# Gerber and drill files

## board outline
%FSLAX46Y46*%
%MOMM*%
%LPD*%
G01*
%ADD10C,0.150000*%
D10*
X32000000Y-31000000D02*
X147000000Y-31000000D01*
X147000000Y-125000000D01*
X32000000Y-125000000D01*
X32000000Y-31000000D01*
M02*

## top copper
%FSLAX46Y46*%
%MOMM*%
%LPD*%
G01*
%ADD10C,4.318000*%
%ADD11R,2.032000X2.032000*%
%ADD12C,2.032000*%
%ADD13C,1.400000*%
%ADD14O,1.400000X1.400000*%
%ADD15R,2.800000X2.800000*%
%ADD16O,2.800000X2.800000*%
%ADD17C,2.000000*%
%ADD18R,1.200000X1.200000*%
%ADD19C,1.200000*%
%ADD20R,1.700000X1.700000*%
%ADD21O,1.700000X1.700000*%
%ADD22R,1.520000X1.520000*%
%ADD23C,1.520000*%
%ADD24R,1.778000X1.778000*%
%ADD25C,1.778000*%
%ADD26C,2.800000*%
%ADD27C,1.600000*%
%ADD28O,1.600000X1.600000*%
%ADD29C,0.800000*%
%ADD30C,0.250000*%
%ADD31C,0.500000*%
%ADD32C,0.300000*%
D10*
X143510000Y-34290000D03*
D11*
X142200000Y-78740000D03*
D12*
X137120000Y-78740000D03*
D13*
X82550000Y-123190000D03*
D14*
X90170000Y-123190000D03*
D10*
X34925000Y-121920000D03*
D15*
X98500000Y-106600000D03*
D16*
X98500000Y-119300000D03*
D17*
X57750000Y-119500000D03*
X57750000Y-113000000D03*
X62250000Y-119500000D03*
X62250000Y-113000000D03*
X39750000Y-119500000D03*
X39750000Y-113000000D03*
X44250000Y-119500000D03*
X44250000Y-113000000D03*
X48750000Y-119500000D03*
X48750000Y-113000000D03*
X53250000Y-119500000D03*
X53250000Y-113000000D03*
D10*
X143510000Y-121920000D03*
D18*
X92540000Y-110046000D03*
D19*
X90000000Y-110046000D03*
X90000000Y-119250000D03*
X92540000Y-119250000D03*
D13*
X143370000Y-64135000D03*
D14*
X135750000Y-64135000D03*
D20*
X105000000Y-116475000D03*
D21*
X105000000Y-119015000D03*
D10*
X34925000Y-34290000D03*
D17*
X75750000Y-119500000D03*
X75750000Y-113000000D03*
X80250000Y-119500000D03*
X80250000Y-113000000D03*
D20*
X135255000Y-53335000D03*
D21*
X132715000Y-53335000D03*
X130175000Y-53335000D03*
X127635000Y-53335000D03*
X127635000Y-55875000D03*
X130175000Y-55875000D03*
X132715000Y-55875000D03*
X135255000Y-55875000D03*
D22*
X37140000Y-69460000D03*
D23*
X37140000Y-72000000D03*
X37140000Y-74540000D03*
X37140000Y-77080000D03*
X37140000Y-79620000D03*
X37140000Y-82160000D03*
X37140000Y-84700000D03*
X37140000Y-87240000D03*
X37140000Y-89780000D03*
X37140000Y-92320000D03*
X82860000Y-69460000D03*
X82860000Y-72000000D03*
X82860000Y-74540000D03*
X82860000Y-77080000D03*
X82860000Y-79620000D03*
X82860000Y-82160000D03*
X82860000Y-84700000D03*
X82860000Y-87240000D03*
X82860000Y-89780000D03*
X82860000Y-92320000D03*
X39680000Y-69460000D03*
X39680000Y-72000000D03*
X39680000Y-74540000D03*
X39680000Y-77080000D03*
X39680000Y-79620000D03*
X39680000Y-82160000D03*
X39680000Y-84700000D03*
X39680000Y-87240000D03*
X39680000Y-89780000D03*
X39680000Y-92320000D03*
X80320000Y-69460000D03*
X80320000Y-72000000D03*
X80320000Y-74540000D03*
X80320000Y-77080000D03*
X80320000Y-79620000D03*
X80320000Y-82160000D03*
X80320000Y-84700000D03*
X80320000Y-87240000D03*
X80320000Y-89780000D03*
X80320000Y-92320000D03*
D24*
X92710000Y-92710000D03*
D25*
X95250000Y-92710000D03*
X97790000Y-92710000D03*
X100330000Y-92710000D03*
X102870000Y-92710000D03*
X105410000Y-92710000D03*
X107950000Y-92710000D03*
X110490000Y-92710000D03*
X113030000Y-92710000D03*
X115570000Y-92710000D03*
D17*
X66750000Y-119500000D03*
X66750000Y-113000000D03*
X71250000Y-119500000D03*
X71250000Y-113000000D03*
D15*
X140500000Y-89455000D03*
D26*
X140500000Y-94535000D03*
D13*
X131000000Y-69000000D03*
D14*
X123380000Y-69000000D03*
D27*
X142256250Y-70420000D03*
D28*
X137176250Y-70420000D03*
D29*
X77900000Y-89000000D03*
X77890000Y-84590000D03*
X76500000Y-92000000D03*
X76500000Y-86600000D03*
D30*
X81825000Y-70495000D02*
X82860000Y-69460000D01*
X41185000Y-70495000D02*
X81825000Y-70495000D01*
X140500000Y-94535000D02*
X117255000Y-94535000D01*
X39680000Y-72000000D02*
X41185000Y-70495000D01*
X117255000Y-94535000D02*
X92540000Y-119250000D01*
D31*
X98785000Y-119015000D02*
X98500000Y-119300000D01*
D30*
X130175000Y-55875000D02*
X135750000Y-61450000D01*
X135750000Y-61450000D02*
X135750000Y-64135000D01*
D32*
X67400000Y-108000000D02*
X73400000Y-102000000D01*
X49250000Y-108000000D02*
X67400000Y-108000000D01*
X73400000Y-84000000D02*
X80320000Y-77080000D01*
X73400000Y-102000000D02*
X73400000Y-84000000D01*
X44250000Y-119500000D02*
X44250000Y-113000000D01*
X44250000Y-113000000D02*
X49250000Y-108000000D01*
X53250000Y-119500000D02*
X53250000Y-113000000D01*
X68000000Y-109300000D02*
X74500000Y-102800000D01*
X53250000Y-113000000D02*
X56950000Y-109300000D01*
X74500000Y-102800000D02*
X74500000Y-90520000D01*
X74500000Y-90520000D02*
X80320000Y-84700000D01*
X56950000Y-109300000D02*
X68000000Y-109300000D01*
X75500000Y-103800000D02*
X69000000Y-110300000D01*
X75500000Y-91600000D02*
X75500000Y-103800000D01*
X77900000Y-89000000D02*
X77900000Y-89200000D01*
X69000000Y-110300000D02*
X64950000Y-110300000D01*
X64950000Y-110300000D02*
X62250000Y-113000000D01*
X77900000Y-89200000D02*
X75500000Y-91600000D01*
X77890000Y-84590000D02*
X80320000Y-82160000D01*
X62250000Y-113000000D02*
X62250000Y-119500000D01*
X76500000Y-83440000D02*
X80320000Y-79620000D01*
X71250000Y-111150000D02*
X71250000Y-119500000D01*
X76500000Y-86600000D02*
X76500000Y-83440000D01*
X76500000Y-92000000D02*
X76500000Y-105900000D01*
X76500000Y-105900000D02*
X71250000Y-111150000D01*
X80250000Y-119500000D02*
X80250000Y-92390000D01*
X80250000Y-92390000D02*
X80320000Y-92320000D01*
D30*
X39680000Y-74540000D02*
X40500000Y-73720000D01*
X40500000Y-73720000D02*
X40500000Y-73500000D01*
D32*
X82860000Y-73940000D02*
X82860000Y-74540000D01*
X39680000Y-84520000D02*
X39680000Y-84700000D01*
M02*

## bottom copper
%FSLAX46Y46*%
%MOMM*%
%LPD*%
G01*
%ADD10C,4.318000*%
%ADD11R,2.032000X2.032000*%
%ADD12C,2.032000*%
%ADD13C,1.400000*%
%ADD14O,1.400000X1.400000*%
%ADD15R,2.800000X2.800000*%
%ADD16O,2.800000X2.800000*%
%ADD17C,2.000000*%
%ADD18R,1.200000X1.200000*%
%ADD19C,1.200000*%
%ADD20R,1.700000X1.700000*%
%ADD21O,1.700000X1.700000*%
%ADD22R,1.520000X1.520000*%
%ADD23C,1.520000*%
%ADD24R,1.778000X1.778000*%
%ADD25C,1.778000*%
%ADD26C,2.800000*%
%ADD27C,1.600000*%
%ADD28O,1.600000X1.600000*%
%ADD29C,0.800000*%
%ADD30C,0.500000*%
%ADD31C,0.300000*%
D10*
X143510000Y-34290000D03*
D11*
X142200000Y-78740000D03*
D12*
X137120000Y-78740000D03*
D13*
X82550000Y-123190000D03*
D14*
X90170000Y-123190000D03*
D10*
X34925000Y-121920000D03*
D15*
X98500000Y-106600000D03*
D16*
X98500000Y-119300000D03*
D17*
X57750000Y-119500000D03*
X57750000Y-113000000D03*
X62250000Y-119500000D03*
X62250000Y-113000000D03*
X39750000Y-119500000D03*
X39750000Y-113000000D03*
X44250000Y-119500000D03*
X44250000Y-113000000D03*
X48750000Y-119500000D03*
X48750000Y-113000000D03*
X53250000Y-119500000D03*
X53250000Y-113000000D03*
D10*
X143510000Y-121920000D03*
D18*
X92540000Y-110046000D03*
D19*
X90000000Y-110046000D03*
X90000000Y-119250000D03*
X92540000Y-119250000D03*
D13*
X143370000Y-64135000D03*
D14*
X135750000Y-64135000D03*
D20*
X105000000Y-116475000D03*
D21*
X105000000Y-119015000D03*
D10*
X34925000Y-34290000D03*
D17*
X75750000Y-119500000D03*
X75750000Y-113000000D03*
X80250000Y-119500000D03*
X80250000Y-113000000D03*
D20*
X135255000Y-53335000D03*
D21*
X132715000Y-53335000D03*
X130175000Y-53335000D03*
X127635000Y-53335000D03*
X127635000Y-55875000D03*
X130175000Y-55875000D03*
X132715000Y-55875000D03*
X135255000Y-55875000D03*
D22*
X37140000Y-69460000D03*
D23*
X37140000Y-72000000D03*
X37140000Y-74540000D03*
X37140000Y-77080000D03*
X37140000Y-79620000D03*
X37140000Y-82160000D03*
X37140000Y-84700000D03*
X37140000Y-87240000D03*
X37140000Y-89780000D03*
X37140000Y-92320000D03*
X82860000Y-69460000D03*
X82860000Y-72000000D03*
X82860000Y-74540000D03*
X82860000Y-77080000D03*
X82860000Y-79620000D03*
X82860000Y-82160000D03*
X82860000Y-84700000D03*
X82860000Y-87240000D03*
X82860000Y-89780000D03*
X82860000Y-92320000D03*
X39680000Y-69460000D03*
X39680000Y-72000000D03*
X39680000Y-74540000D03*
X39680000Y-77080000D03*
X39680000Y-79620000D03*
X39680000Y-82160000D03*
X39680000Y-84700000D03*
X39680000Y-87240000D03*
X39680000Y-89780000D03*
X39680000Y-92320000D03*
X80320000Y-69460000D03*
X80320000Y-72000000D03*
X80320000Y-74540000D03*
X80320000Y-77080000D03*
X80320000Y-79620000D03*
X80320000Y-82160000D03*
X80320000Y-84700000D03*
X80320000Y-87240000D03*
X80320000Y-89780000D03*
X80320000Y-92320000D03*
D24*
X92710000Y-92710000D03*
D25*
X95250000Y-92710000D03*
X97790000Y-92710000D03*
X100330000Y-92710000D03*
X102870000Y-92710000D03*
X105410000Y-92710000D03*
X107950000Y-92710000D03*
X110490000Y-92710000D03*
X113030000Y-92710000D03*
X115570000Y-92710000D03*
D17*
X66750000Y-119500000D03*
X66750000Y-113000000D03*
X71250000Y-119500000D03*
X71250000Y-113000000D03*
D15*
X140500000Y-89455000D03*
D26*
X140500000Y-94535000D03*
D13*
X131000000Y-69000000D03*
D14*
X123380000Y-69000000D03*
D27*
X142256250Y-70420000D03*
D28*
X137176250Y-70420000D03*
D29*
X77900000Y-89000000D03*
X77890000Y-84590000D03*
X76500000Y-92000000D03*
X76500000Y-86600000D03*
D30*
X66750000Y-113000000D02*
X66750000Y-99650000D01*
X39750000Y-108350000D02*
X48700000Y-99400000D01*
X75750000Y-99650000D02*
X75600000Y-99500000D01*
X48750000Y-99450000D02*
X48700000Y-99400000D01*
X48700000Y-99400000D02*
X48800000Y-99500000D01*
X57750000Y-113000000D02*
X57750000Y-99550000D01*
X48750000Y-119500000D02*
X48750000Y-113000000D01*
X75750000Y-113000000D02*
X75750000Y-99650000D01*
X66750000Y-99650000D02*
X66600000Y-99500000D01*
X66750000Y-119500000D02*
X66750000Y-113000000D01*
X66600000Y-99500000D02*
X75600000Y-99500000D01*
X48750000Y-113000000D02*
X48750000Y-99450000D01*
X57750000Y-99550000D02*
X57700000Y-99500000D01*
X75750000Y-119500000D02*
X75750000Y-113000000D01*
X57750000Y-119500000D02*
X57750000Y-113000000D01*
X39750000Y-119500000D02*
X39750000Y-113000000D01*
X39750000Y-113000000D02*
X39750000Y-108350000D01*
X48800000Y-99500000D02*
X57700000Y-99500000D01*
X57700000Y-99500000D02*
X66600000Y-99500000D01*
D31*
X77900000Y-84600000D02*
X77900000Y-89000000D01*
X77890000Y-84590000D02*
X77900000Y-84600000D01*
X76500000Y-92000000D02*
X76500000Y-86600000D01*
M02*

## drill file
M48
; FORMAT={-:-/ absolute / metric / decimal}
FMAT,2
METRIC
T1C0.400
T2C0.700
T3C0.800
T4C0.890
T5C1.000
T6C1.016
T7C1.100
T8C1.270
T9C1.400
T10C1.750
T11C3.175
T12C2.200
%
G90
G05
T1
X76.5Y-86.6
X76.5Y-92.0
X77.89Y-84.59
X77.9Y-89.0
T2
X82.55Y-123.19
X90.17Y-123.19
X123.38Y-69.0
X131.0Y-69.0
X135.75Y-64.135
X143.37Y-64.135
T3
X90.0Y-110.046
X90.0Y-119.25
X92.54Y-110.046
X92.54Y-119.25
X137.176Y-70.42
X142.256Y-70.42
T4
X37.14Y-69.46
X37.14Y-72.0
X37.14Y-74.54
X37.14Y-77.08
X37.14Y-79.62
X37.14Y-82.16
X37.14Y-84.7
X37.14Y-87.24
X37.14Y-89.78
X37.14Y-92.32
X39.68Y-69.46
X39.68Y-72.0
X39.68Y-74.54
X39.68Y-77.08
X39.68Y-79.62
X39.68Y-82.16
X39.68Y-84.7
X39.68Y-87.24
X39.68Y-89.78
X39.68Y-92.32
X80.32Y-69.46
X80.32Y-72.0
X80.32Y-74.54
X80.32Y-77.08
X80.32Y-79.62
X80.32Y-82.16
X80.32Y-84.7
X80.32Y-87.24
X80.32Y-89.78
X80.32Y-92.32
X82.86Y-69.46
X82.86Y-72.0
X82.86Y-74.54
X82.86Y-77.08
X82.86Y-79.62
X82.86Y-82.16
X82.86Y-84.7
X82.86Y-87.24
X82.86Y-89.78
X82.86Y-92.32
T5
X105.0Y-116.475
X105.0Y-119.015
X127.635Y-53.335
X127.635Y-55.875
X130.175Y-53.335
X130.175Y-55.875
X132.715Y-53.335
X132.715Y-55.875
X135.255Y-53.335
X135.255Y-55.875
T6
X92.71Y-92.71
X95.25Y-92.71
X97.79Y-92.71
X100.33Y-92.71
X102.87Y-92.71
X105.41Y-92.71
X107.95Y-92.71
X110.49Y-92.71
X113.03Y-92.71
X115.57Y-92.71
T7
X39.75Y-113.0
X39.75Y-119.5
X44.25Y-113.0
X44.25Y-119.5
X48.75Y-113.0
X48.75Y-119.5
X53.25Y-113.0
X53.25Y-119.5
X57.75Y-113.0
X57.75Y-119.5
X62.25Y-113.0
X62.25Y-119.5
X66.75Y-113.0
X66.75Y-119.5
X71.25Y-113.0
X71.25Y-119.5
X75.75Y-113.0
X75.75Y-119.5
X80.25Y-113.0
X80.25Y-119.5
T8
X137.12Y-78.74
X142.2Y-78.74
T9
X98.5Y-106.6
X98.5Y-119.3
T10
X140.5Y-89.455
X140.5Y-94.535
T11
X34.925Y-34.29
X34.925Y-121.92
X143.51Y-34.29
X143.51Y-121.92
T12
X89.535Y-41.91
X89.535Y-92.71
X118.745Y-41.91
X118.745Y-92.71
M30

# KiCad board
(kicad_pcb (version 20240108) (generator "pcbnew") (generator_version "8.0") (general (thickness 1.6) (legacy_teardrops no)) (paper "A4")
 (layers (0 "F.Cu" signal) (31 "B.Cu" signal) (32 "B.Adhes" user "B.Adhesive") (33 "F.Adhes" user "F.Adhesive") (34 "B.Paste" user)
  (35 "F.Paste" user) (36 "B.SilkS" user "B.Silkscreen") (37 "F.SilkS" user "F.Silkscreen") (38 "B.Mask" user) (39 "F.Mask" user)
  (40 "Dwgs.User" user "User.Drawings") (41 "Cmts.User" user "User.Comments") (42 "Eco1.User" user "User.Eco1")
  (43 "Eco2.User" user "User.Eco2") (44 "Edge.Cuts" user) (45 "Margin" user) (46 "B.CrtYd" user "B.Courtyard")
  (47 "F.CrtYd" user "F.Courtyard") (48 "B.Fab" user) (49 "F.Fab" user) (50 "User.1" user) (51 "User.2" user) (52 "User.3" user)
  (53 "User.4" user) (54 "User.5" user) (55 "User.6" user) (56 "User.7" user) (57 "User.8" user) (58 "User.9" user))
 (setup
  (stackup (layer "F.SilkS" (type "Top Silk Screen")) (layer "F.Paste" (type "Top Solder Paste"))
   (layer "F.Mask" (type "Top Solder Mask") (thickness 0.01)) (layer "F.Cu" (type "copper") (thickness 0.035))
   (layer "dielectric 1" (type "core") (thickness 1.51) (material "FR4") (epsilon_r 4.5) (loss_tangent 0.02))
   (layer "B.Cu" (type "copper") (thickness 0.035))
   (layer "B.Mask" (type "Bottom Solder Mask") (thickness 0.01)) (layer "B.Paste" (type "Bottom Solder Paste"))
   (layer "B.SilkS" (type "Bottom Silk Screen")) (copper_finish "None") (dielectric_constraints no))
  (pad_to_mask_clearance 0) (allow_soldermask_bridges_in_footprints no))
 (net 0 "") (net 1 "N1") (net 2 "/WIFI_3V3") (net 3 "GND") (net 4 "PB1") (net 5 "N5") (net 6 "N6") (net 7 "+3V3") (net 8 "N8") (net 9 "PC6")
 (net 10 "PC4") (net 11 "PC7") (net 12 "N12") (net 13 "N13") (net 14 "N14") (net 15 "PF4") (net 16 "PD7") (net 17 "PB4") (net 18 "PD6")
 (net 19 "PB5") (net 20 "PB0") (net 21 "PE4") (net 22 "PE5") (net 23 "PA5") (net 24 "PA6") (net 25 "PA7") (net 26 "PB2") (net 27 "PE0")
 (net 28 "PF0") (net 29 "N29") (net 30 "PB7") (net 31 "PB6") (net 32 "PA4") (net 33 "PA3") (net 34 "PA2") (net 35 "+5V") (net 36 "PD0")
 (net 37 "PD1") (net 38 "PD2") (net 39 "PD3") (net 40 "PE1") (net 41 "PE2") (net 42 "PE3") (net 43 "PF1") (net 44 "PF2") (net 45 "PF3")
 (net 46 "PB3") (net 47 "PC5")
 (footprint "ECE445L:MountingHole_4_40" (layer "F.Cu") (at 143.51 34.29)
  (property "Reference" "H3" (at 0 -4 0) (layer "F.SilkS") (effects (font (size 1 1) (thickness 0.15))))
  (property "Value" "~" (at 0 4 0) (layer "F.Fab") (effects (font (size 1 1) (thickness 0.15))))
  (pad "1" thru_hole circle (at 0 0) (size 4.318 4.318) (drill 3.175) (layers "*.Cu" "*.Mask") (remove_unused_layers no) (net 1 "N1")))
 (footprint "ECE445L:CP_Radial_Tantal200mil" (layer "F.Cu") (at 142.2 78.74 180)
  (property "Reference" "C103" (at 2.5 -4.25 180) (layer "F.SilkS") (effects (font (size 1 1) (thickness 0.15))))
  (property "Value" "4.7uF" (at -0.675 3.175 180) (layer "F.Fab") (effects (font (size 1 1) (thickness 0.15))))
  (pad "1" thru_hole rect (at 0 0 180) (size 2.032 2.032) (drill 1.27) (layers "*.Cu" "*.Mask") (remove_unused_layers no)
   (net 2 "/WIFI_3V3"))
  (pad "2" thru_hole circle (at 5.08 0 180) (size 2.032 2.032) (drill 1.27) (layers "*.Cu" "*.Mask") (remove_unused_layers no) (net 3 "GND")))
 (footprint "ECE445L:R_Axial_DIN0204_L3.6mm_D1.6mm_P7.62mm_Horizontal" (layer "F.Cu") (at 82.55 123.19)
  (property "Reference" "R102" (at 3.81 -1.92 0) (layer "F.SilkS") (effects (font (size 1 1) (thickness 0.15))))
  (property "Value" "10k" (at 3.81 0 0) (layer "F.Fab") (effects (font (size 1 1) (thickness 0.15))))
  (pad "1" thru_hole circle (at 0 0) (size 1.4 1.4) (drill 0.7) (layers "*.Cu" "*.Mask") (remove_unused_layers no) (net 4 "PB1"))
  (pad "2" thru_hole oval (at 7.62 0) (size 1.4 1.4) (drill 0.7) (layers "*.Cu" "*.Mask") (remove_unused_layers no) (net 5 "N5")))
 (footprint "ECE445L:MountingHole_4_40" (layer "F.Cu") (at 34.925 121.92)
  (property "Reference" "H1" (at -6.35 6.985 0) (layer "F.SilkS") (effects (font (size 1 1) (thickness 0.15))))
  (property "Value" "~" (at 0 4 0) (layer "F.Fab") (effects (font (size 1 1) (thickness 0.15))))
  (pad "1" thru_hole circle (at 0 0) (size 4.318 4.318) (drill 3.175) (layers "*.Cu" "*.Mask") (remove_unused_layers no) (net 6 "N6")))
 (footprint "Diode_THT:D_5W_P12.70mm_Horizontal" (layer "F.Cu") (at 98.5 106.6 -90)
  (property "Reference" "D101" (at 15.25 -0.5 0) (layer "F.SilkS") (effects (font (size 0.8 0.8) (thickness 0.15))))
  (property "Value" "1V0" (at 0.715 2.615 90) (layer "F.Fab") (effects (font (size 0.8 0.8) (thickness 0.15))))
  (pad "1" thru_hole rect (at 0 0 270) (size 2.8 2.8) (drill 1.4) (layers "*.Cu" "*.Mask") (remove_unused_layers no) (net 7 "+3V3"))
  (pad "2" thru_hole oval (at 12.7 0 270) (size 2.8 2.8) (drill 1.4) (layers "*.Cu" "*.Mask") (remove_unused_layers no) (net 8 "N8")))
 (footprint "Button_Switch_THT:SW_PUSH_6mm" (layer "F.Cu") (at 57.75 119.5 90)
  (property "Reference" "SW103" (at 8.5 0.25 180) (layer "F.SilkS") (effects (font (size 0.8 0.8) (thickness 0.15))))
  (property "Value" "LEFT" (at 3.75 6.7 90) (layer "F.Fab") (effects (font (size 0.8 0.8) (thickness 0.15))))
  (pad "1" thru_hole circle (at 0 0 180) (size 2 2) (drill 1.1) (layers "*.Cu" "*.Mask") (remove_unused_layers no) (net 3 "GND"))
  (pad "1" thru_hole circle (at 6.5 0 180) (size 2 2) (drill 1.1) (layers "*.Cu" "*.Mask") (remove_unused_layers no) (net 3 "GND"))
  (pad "2" thru_hole circle (at 0 4.5 180) (size 2 2) (drill 1.1) (layers "*.Cu" "*.Mask") (remove_unused_layers no) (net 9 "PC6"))
  (pad "2" thru_hole circle (at 6.5 4.5 180) (size 2 2) (drill 1.1) (layers "*.Cu" "*.Mask") (remove_unused_layers no) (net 9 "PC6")))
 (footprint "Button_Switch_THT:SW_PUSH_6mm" (layer "F.Cu") (at 39.75 119.5 90)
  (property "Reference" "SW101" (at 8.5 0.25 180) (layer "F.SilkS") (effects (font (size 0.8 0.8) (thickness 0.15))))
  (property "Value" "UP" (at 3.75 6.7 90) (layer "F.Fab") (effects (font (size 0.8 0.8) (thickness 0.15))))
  (pad "1" thru_hole circle (at 0 0 180) (size 2 2) (drill 1.1) (layers "*.Cu" "*.Mask") (remove_unused_layers no) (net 3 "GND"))
  (pad "1" thru_hole circle (at 6.5 0 180) (size 2 2) (drill 1.1) (layers "*.Cu" "*.Mask") (remove_unused_layers no) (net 3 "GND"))
  (pad "2" thru_hole circle (at 0 4.5 180) (size 2 2) (drill 1.1) (layers "*.Cu" "*.Mask") (remove_unused_layers no) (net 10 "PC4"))
  (pad "2" thru_hole circle (at 6.5 4.5 180) (size 2 2) (drill 1.1) (layers "*.Cu" "*.Mask") (remove_unused_layers no) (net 10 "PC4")))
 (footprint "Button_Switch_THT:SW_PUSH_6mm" (layer "F.Cu") (at 48.75 119.5 90)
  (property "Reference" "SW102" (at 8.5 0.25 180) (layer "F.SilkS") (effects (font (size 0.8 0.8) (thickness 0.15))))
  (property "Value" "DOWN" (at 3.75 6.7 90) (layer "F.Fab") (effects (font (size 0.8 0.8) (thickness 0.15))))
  (pad "1" thru_hole circle (at 0 0 180) (size 2 2) (drill 1.1) (layers "*.Cu" "*.Mask") (remove_unused_layers no) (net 3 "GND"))
  (pad "1" thru_hole circle (at 6.5 0 180) (size 2 2) (drill 1.1) (layers "*.Cu" "*.Mask") (remove_unused_layers no) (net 3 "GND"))
  (pad "2" thru_hole circle (at 0 4.5 180) (size 2 2) (drill 1.1) (layers "*.Cu" "*.Mask") (remove_unused_layers no) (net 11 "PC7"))
  (pad "2" thru_hole circle (at 6.5 4.5 180) (size 2 2) (drill 1.1) (layers "*.Cu" "*.Mask") (remove_unused_layers no) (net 11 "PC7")))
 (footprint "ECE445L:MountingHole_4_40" (layer "F.Cu") (at 143.51 121.92)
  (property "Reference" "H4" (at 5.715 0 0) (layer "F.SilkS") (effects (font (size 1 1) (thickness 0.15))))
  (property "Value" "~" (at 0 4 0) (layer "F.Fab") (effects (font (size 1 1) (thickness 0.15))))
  (pad "1" thru_hole circle (at 0 0) (size 4.318 4.318) (drill 3.175) (layers "*.Cu" "*.Mask") (remove_unused_layers no) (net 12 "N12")))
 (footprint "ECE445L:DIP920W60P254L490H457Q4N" (layer "F.Cu") (at 91.27 114.648 -90)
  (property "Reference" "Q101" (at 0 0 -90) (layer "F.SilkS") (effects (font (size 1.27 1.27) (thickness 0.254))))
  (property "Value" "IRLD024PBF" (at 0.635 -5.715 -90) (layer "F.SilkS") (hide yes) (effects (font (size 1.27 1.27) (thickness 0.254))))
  (pad "1" thru_hole rect (at -4.602 -1.27 270) (size 1.2 1.2) (drill 0.8) (layers "*.Cu" "*.Mask") (remove_unused_layers no) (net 8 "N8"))
  (pad "2" thru_hole circle (at -4.602 1.27 270) (size 1.2 1.2) (drill 0.8) (layers "*.Cu" "*.Mask") (remove_unused_layers no) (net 8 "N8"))
  (pad "3" thru_hole circle (at 4.602 1.27 270) (size 1.2 1.2) (drill 0.8) (layers "*.Cu" "*.Mask") (remove_unused_layers no) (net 5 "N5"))
  (pad "4" thru_hole circle (at 4.602 -1.27 270) (size 1.2 1.2) (drill 0.8) (layers "*.Cu" "*.Mask") (remove_unused_layers no) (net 3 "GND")))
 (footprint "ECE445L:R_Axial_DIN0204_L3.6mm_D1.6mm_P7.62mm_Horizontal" (layer "F.Cu") (at 143.37 64.135 180)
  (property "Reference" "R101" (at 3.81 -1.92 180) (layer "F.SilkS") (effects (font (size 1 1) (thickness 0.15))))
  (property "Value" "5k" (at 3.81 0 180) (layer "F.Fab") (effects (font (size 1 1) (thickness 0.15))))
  (pad "1" thru_hole circle (at 0 0 180) (size 1.4 1.4) (drill 0.7) (layers "*.Cu" "*.Mask") (remove_unused_layers no) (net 2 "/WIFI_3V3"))
  (pad "2" thru_hole oval (at 7.62 0 180) (size 1.4 1.4) (drill 0.7) (layers "*.Cu" "*.Mask") (remove_unused_layers no) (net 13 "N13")))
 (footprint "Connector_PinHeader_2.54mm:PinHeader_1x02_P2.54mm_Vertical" (layer "F.Cu") (at 105 116.475)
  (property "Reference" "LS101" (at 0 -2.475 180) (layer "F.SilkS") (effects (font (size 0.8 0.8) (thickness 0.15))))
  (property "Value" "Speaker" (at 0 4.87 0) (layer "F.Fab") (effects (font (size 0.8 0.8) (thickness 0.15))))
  (pad "1" thru_hole rect (at 0 0) (size 1.7 1.7) (drill 1) (layers "*.Cu" "*.Mask") (remove_unused_layers no) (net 7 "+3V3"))
  (pad "2" thru_hole oval (at 0 2.54) (size 1.7 1.7) (drill 1) (layers "*.Cu" "*.Mask") (remove_unused_layers no) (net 8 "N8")))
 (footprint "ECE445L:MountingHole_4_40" (layer "F.Cu") (at 34.925 34.29)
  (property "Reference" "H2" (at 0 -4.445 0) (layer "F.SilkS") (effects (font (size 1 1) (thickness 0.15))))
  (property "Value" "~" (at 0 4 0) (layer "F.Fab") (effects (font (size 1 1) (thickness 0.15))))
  (pad "1" thru_hole circle (at 0 0) (size 4.318 4.318) (drill 3.175) (layers "*.Cu" "*.Mask") (remove_unused_layers no) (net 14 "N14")))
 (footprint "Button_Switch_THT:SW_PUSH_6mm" (layer "F.Cu") (at 75.75 119.5 90)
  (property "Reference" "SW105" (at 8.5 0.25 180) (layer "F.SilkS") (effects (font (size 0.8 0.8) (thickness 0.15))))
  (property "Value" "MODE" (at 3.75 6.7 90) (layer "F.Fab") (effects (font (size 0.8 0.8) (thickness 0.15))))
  (pad "1" thru_hole circle (at 0 0 180) (size 2 2) (drill 1.1) (layers "*.Cu" "*.Mask") (remove_unused_layers no) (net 3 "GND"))
  (pad "1" thru_hole circle (at 6.5 0 180) (size 2 2) (drill 1.1) (layers "*.Cu" "*.Mask") (remove_unused_layers no) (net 3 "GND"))
  (pad "2" thru_hole circle (at 0 4.5 180) (size 2 2) (drill 1.1) (layers "*.Cu" "*.Mask") (remove_unused_layers no) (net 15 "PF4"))
  (pad "2" thru_hole circle (at 6.5 4.5 180) (size 2 2) (drill 1.1) (layers "*.Cu" "*.Mask") (remove_unused_layers no) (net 15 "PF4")))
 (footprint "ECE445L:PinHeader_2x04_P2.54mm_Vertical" (layer "F.Cu") (at 135.255 53.335 -90)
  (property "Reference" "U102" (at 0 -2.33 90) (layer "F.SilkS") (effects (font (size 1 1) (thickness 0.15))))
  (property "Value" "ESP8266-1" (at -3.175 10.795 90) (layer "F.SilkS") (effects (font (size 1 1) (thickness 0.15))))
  (pad "1" thru_hole rect (at 0 0 270) (size 1.7 1.7) (drill 1) (layers "*.Cu" "*.Mask") (remove_unused_layers no) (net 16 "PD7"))
  (pad "2" thru_hole oval (at 0 2.54 270) (size 1.7 1.7) (drill 1) (layers "*.Cu" "*.Mask") (remove_unused_layers no) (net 2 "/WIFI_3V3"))
  (pad "3" thru_hole oval (at 0 5.08 270) (size 1.7 1.7) (drill 1) (layers "*.Cu" "*.Mask") (remove_unused_layers no) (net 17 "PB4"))
  (pad "4" thru_hole oval (at 0 7.62 270) (size 1.7 1.7) (drill 1) (layers "*.Cu" "*.Mask") (remove_unused_layers no) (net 3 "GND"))
  (pad "5" thru_hole oval (at 2.54 7.62 270) (size 1.7 1.7) (drill 1) (layers "*.Cu" "*.Mask") (remove_unused_layers no) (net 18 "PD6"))
  (pad "6" thru_hole oval (at 2.54 5.08 270) (size 1.7 1.7) (drill 1) (layers "*.Cu" "*.Mask") (remove_unused_layers no) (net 13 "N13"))
  (pad "7" thru_hole oval (at 2.54 2.54 270) (size 1.7 1.7) (drill 1) (layers "*.Cu" "*.Mask") (remove_unused_layers no) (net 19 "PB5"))
  (pad "8" thru_hole oval (at 2.54 0 270) (size 1.7 1.7) (drill 1) (layers "*.Cu" "*.Mask") (remove_unused_layers no) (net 2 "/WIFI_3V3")))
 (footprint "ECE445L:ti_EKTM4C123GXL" (layer "F.Cu") (at 60 72)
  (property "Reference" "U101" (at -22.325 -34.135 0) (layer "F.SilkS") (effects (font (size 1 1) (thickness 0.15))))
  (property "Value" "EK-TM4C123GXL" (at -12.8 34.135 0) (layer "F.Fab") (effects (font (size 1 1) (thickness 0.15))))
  (pad "J1_1" thru_hole rect (at -22.86 -2.54) (size 1.52 1.52) (drill 0.89) (layers "*.Cu" "*.Mask") (remove_unused_layers no)
   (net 7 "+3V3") (solder_mask_margin 0.102))
  (pad "J1_2" thru_hole circle (at -22.86 0) (size 1.52 1.52) (drill 0.89) (layers "*.Cu" "*.Mask") (remove_unused_layers no) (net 19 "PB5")
   (solder_mask_margin 0.102))
  (pad "J1_3" thru_hole circle (at -22.86 2.54) (size 1.52 1.52) (drill 0.89) (layers "*.Cu" "*.Mask") (remove_unused_layers no)
   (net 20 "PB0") (solder_mask_margin 0.102))
  (pad "J1_4" thru_hole circle (at -22.86 5.08) (size 1.52 1.52) (drill 0.89) (layers "*.Cu" "*.Mask") (remove_unused_layers no)
   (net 4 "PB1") (solder_mask_margin 0.102))
  (pad "J1_5" thru_hole circle (at -22.86 7.62) (size 1.52 1.52) (drill 0.89) (layers "*.Cu" "*.Mask") (remove_unused_layers no)
   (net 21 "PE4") (solder_mask_margin 0.102))
  (pad "J1_6" thru_hole circle (at -22.86 10.16) (size 1.52 1.52) (drill 0.89) (layers "*.Cu" "*.Mask") (remove_unused_layers no)
   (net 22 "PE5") (solder_mask_margin 0.102))
  (pad "J1_7" thru_hole circle (at -22.86 12.7) (size 1.52 1.52) (drill 0.89) (layers "*.Cu" "*.Mask") (remove_unused_layers no)
   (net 17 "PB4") (solder_mask_margin 0.102))
  (pad "J1_8" thru_hole circle (at -22.86 15.24) (size 1.52 1.52) (drill 0.89) (layers "*.Cu" "*.Mask") (remove_unused_layers no)
   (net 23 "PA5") (solder_mask_margin 0.102))
  (pad "J1_9" thru_hole circle (at -22.86 17.78) (size 1.52 1.52) (drill 0.89) (layers "*.Cu" "*.Mask") (remove_unused_layers no)
   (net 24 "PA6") (solder_mask_margin 0.102))
  (pad "J1_10" thru_hole circle (at -22.86 20.32) (size 1.52 1.52) (drill 0.89) (layers "*.Cu" "*.Mask") (remove_unused_layers no)
   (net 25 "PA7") (solder_mask_margin 0.102))
  (pad "J2_1" thru_hole circle (at 22.86 -2.54) (size 1.52 1.52) (drill 0.89) (layers "*.Cu" "*.Mask") (remove_unused_layers no)
   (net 3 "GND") (solder_mask_margin 0.102))
  (pad "J2_2" thru_hole circle (at 22.86 0) (size 1.52 1.52) (drill 0.89) (layers "*.Cu" "*.Mask") (remove_unused_layers no) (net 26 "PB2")
   (solder_mask_margin 0.102))
  (pad "J2_3" thru_hole circle (at 22.86 2.54) (size 1.52 1.52) (drill 0.89) (layers "*.Cu" "*.Mask") (remove_unused_layers no)
   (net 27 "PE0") (solder_mask_margin 0.102))
  (pad "J2_4" thru_hole circle (at 22.86 5.08) (size 1.52 1.52) (drill 0.89) (layers "*.Cu" "*.Mask") (remove_unused_layers no)
   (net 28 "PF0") (solder_mask_margin 0.102))
  (pad "J2_5" thru_hole circle (at 22.86 7.62) (size 1.52 1.52) (drill 0.89) (layers "*.Cu" "*.Mask") (remove_unused_layers no)
   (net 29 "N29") (solder_mask_margin 0.102))
  (pad "J2_6" thru_hole circle (at 22.86 10.16) (size 1.52 1.52) (drill 0.89) (layers "*.Cu" "*.Mask") (remove_unused_layers no)
   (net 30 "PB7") (solder_mask_margin 0.102))
  (pad "J2_7" thru_hole circle (at 22.86 12.7) (size 1.52 1.52) (drill 0.89) (layers "*.Cu" "*.Mask") (remove_unused_layers no)
   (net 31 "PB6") (solder_mask_margin 0.102))
  (pad "J2_8" thru_hole circle (at 22.86 15.24) (size 1.52 1.52) (drill 0.89) (layers "*.Cu" "*.Mask") (remove_unused_layers no)
   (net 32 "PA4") (solder_mask_margin 0.102))
  (pad "J2_9" thru_hole circle (at 22.86 17.78) (size 1.52 1.52) (drill 0.89) (layers "*.Cu" "*.Mask") (remove_unused_layers no)
   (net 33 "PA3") (solder_mask_margin 0.102))
  (pad "J2_10" thru_hole circle (at 22.86 20.32) (size 1.52 1.52) (drill 0.89) (layers "*.Cu" "*.Mask") (remove_unused_layers no)
   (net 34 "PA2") (solder_mask_margin 0.102))
  (pad "J3_1" thru_hole circle (at -20.32 -2.54) (size 1.52 1.52) (drill 0.89) (layers "*.Cu" "*.Mask") (remove_unused_layers no)
   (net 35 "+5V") (solder_mask_margin 0.102))
  (pad "J3_2" thru_hole circle (at -20.32 0) (size 1.52 1.52) (drill 0.89) (layers "*.Cu" "*.Mask") (remove_unused_layers no) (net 3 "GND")
   (solder_mask_margin 0.102))
  (pad "J3_3" thru_hole circle (at -20.32 2.54) (size 1.52 1.52) (drill 0.89) (layers "*.Cu" "*.Mask") (remove_unused_layers no)
   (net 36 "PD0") (solder_mask_margin 0.102))
  (pad "J3_4" thru_hole circle (at -20.32 5.08) (size 1.52 1.52) (drill 0.89) (layers "*.Cu" "*.Mask") (remove_unused_layers no)
   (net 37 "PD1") (solder_mask_margin 0.102))
  (pad "J3_5" thru_hole circle (at -20.32 7.62) (size 1.52 1.52) (drill 0.89) (layers "*.Cu" "*.Mask") (remove_unused_layers no)
   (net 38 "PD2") (solder_mask_margin 0.102))
  (pad "J3_6" thru_hole circle (at -20.32 10.16) (size 1.52 1.52) (drill 0.89) (layers "*.Cu" "*.Mask") (remove_unused_layers no)
   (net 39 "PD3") (solder_mask_margin 0.102))
  (pad "J3_7" thru_hole circle (at -20.32 12.7) (size 1.52 1.52) (drill 0.89) (layers "*.Cu" "*.Mask") (remove_unused_layers no)
   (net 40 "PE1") (solder_mask_margin 0.102))
  (pad "J3_8" thru_hole circle (at -20.32 15.24) (size 1.52 1.52) (drill 0.89) (layers "*.Cu" "*.Mask") (remove_unused_layers no)
   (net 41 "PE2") (solder_mask_margin 0.102))
  (pad "J3_9" thru_hole circle (at -20.32 17.78) (size 1.52 1.52) (drill 0.89) (layers "*.Cu" "*.Mask") (remove_unused_layers no)
   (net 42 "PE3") (solder_mask_margin 0.102))
  (pad "J3_10" thru_hole circle (at -20.32 20.32) (size 1.52 1.52) (drill 0.89) (layers "*.Cu" "*.Mask") (remove_unused_layers no)
   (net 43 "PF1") (solder_mask_margin 0.102))
  (pad "J4_1" thru_hole circle (at 20.32 -2.54) (size 1.52 1.52) (drill 0.89) (layers "*.Cu" "*.Mask") (remove_unused_layers no)
   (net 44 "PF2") (solder_mask_margin 0.102))
  (pad "J4_2" thru_hole circle (at 20.32 0) (size 1.52 1.52) (drill 0.89) (layers "*.Cu" "*.Mask") (remove_unused_layers no) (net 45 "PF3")
   (solder_mask_margin 0.102))
  (pad "J4_3" thru_hole circle (at 20.32 2.54) (size 1.52 1.52) (drill 0.89) (layers "*.Cu" "*.Mask") (remove_unused_layers no)
   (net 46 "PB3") (solder_mask_margin 0.102))
  (pad "J4_4" thru_hole circle (at 20.32 5.08) (size 1.52 1.52) (drill 0.89) (layers "*.Cu" "*.Mask") (remove_unused_layers no)
   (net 10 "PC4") (solder_mask_margin 0.102))
  (pad "J4_5" thru_hole circle (at 20.32 7.62) (size 1.52 1.52) (drill 0.89) (layers "*.Cu" "*.Mask") (remove_unused_layers no)
   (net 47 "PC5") (solder_mask_margin 0.102))
  (pad "J4_6" thru_hole circle (at 20.32 10.16) (size 1.52 1.52) (drill 0.89) (layers "*.Cu" "*.Mask") (remove_unused_layers no)
   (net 9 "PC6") (solder_mask_margin 0.102))
  (pad "J4_7" thru_hole circle (at 20.32 12.7) (size 1.52 1.52) (drill 0.89) (layers "*.Cu" "*.Mask") (remove_unused_layers no)
   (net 11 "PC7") (solder_mask_margin 0.102))
  (pad "J4_8" thru_hole circle (at 20.32 15.24) (size 1.52 1.52) (drill 0.89) (layers "*.Cu" "*.Mask") (remove_unused_layers no)
   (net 18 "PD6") (solder_mask_margin 0.102))
  (pad "J4_9" thru_hole circle (at 20.32 17.78) (size 1.52 1.52) (drill 0.89) (layers "*.Cu" "*.Mask") (remove_unused_layers no)
   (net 16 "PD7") (solder_mask_margin 0.102))
  (pad "J4_10" thru_hole circle (at 20.32 20.32) (size 1.52 1.52) (drill 0.89) (layers "*.Cu" "*.Mask") (remove_unused_layers no)
   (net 15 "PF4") (solder_mask_margin 0.102)))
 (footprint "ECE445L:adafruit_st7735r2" (layer "F.Cu") (at 104.14 67.31)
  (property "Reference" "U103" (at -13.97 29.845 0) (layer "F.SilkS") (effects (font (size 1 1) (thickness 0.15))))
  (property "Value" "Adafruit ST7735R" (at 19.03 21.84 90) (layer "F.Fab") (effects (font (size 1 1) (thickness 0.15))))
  (pad "" np_thru_hole circle (at -14.605 -25.4 90) (size 2.2 2.2) (drill 2.2) (layers "*.Cu" "*.Mask"))
  (pad "" np_thru_hole circle (at -14.605 25.4 90) (size 2.2 2.2) (drill 2.2) (layers "F&B.Cu" "*.Mask"))
  (pad "" np_thru_hole circle (at 14.605 -25.4 90) (size 2.2 2.2) (drill 2.2) (layers "F&B.Cu" "*.Mask"))
  (pad "" np_thru_hole circle (at 14.605 25.4 90) (size 2.2 2.2) (drill 2.2) (layers "F&B.Cu" "*.Mask"))
  (pad "1" thru_hole rect (at -11.43 25.4 90) (size 1.778 1.778) (drill 1.016) (layers "*.Cu" "*.Mask") (remove_unused_layers no)
   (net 3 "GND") (solder_mask_margin 0.102))
  (pad "2" thru_hole circle (at -8.89 25.4 90) (size 1.778 1.778) (drill 1.016) (layers "*.Cu" "*.Mask") (remove_unused_layers no)
   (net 7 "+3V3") (solder_mask_margin 0.102))
  (pad "3" thru_hole circle (at -6.35 25.4 90) (size 1.778 1.778) (drill 1.016) (layers "*.Cu" "*.Mask") (remove_unused_layers no)
   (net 25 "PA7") (solder_mask_margin 0.102))
  (pad "4" thru_hole circle (at -3.81 25.4 90) (size 1.778 1.778) (drill 1.016) (layers "*.Cu" "*.Mask") (remove_unused_layers no)
   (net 24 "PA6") (solder_mask_margin 0.102))
  (pad "5" thru_hole circle (at -1.27 25.4 90) (size 1.778 1.778) (drill 1.016) (layers "*.Cu" "*.Mask") (remove_unused_layers no)
   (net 20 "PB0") (solder_mask_margin 0.102))
  (pad "6" thru_hole circle (at 1.27 25.4 90) (size 1.778 1.778) (drill 1.016) (layers "*.Cu" "*.Mask") (remove_unused_layers no)
   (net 33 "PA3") (solder_mask_margin 0.102))
  (pad "7" thru_hole circle (at 3.81 25.4 90) (size 1.778 1.778) (drill 1.016) (layers "*.Cu" "*.Mask") (remove_unused_layers no)
   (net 23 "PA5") (solder_mask_margin 0.102))
  (pad "8" thru_hole circle (at 6.35 25.4 90) (size 1.778 1.778) (drill 1.016) (layers "*.Cu" "*.Mask") (remove_unused_layers no)
   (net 34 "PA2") (solder_mask_margin 0.102))
  (pad "9" thru_hole circle (at 8.89 25.4 90) (size 1.778 1.778) (drill 1.016) (layers "*.Cu" "*.Mask") (remove_unused_layers no)
   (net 32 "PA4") (solder_mask_margin 0.102))
  (pad "10" thru_hole circle (at 11.43 25.4 90) (size 1.778 1.778) (drill 1.016) (layers "*.Cu" "*.Mask") (remove_unused_layers no)
   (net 7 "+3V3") (solder_mask_margin 0.102)))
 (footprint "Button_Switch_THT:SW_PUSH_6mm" (layer "F.Cu") (at 66.75 119.5 90)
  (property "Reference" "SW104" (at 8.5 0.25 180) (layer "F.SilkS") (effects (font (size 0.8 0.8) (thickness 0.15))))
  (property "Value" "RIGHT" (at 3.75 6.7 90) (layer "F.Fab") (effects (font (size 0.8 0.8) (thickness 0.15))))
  (pad "1" thru_hole circle (at 0 0 180) (size 2 2) (drill 1.1) (layers "*.Cu" "*.Mask") (remove_unused_layers no) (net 3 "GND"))
  (pad "1" thru_hole circle (at 6.5 0 180) (size 2 2) (drill 1.1) (layers "*.Cu" "*.Mask") (remove_unused_layers no) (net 3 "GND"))
  (pad "2" thru_hole circle (at 0 4.5 180) (size 2 2) (drill 1.1) (layers "*.Cu" "*.Mask") (remove_unused_layers no) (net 47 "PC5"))
  (pad "2" thru_hole circle (at 6.5 4.5 180) (size 2 2) (drill 1.1) (layers "*.Cu" "*.Mask") (remove_unused_layers no) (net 47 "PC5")))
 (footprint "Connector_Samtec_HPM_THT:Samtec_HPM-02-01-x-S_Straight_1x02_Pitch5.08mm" (layer "F.Cu") (at 140.5 89.455)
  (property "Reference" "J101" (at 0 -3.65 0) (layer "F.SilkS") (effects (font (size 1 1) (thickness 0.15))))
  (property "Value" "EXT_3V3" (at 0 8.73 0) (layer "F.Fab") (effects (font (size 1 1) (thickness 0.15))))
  (pad "1" thru_hole rect (at 0 0) (size 2.8 2.8) (drill 1.75) (layers "*.Cu" "*.Mask") (remove_unused_layers no) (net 2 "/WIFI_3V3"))
  (pad "2" thru_hole circle (at 0 5.08) (size 2.8 2.8) (drill 1.75) (layers "*.Cu" "*.Mask") (remove_unused_layers no) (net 3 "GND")))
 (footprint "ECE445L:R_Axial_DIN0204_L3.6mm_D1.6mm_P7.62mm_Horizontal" (layer "F.Cu") (at 131 69 180)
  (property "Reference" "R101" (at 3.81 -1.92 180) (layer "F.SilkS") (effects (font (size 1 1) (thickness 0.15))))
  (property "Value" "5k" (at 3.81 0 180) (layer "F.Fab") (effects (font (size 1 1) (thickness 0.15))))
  (pad "1" thru_hole circle (at 0 0 180) (size 1.4 1.4) (drill 0.7) (layers "*.Cu" "*.Mask") (remove_unused_layers no))
  (pad "2" thru_hole oval (at 7.62 0 180) (size 1.4 1.4) (drill 0.7) (layers "*.Cu" "*.Mask") (remove_unused_layers no)))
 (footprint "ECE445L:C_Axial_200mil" (layer "F.Cu") (at 142.25625 70.42 180)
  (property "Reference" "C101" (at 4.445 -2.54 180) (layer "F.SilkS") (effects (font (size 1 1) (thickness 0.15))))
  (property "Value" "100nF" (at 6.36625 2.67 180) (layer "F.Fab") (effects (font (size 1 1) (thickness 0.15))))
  (pad "1" thru_hole circle (at 0 0 180) (size 1.6 1.6) (drill 0.8) (layers "*.Cu" "*.Mask") (remove_unused_layers no) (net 2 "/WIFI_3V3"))
  (pad "2" thru_hole oval (at 5.08 0 180) (size 1.6 1.6) (drill 0.8) (layers "*.Cu" "*.Mask") (remove_unused_layers no) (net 3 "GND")))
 (gr_rect (start 32 31) (end 147 125) (stroke (width 0.15) (type default)) (fill none) (layer "Edge.Cuts"))
 (segment (start 81.825 70.495) (end 82.86 69.46) (width 0.25) (layer "F.Cu") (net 3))
 (segment (start 41.185 70.495) (end 81.825 70.495) (width 0.25) (layer "F.Cu") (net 3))
 (segment (start 140.5 94.535) (end 117.255 94.535) (width 0.25) (layer "F.Cu") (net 3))
 (segment (start 39.68 72) (end 41.185 70.495) (width 0.25) (layer "F.Cu") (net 3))
 (segment (start 117.255 94.535) (end 92.54 119.25) (width 0.25) (layer "F.Cu") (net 3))
 (segment (start 66.75 113) (end 66.75 99.65) (width 0.5) (layer "B.Cu") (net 3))
 (segment (start 39.75 108.35) (end 48.7 99.4) (width 0.5) (layer "B.Cu") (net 3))
 (segment (start 75.75 99.65) (end 75.6 99.5) (width 0.5) (layer "B.Cu") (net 3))
 (segment (start 48.75 99.45) (end 48.7 99.4) (width 0.5) (layer "B.Cu") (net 3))
 (segment (start 48.7 99.4) (end 48.8 99.5) (width 0.5) (layer "B.Cu") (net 3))
 (segment (start 57.75 113) (end 57.75 99.55) (width 0.5) (layer "B.Cu") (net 3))
 (segment (start 48.75 119.5) (end 48.75 113) (width 0.5) (layer "B.Cu") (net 3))
 (segment (start 75.75 113) (end 75.75 99.65) (width 0.5) (layer "B.Cu") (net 3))
 (segment (start 66.75 99.65) (end 66.6 99.5) (width 0.5) (layer "B.Cu") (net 3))
 (segment (start 66.75 119.5) (end 66.75 113) (width 0.5) (layer "B.Cu") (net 3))
 (segment (start 66.6 99.5) (end 75.6 99.5) (width 0.5) (layer "B.Cu") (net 3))
 (segment (start 48.75 113) (end 48.75 99.45) (width 0.5) (layer "B.Cu") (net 3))
 (segment (start 57.75 99.55) (end 57.7 99.5) (width 0.5) (layer "B.Cu") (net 3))
 (segment (start 75.75 119.5) (end 75.75 113) (width 0.5) (layer "B.Cu") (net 3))
 (segment (start 57.75 119.5) (end 57.75 113) (width 0.5) (layer "B.Cu") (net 3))
 (segment (start 39.75 119.5) (end 39.75 113) (width 0.5) (layer "B.Cu") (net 3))
 (segment (start 39.75 113) (end 39.75 108.35) (width 0.5) (layer "B.Cu") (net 3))
 (segment (start 48.8 99.5) (end 57.7 99.5) (width 0.5) (layer "B.Cu") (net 3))
 (segment (start 57.7 99.5) (end 66.6 99.5) (width 0.5) (layer "B.Cu") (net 3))
 (segment (start 98.785 119.015) (end 98.5 119.3) (width 0.5) (layer "F.Cu") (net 8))
 (segment (start 130.175 55.875) (end 135.75 61.45) (width 0.25) (layer "F.Cu") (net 13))
 (segment (start 135.75 61.45) (end 135.75 64.135) (width 0.25) (layer "F.Cu") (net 13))
 (segment (start 67.4 108) (end 73.4 102) (width 0.3) (layer "F.Cu") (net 10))
 (segment (start 49.25 108) (end 67.4 108) (width 0.3) (layer "F.Cu") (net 10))
 (segment (start 73.4 84) (end 80.32 77.08) (width 0.3) (layer "F.Cu") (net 10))
 (segment (start 73.4 102) (end 73.4 84) (width 0.3) (layer "F.Cu") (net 10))
 (segment (start 44.25 119.5) (end 44.25 113) (width 0.3) (layer "F.Cu") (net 10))
 (segment (start 44.25 113) (end 49.25 108) (width 0.3) (layer "F.Cu") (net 10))
 (segment (start 53.25 119.5) (end 53.25 113) (width 0.3) (layer "F.Cu") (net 11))
 (segment (start 68 109.3) (end 74.5 102.8) (width 0.3) (layer "F.Cu") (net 11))
 (segment (start 53.25 113) (end 56.95 109.3) (width 0.3) (layer "F.Cu") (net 11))
 (segment (start 74.5 102.8) (end 74.5 90.52) (width 0.3) (layer "F.Cu") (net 11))
 (segment (start 74.5 90.52) (end 80.32 84.7) (width 0.3) (layer "F.Cu") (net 11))
 (segment (start 56.95 109.3) (end 68 109.3) (width 0.3) (layer "F.Cu") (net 11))
 (segment (start 75.5 103.8) (end 69 110.3) (width 0.3) (layer "F.Cu") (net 9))
 (segment (start 75.5 91.6) (end 75.5 103.8) (width 0.3) (layer "F.Cu") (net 9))
 (segment (start 77.9 89) (end 77.9 89.2) (width 0.3) (layer "F.Cu") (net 9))
 (segment (start 69 110.3) (end 64.95 110.3) (width 0.3) (layer "F.Cu") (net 9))
 (segment (start 64.95 110.3) (end 62.25 113) (width 0.3) (layer "F.Cu") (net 9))
 (segment (start 77.9 89.2) (end 75.5 91.6) (width 0.3) (layer "F.Cu") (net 9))
 (segment (start 77.89 84.59) (end 80.32 82.16) (width 0.3) (layer "F.Cu") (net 9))
 (segment (start 62.25 113) (end 62.25 119.5) (width 0.3) (layer "F.Cu") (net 9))
 (via (at 77.9 89) (size 0.8) (drill 0.4) (layers "F.Cu" "B.Cu") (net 9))
 (via (at 77.89 84.59) (size 0.8) (drill 0.4) (layers "F.Cu" "B.Cu") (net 9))
 (segment (start 77.9 84.6) (end 77.9 89) (width 0.3) (layer "B.Cu") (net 9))
 (segment (start 77.89 84.59) (end 77.9 84.6) (width 0.3) (layer "B.Cu") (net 9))
 (segment (start 76.5 83.44) (end 80.32 79.62) (width 0.3) (layer "F.Cu") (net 47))
 (segment (start 71.25 111.15) (end 71.25 119.5) (width 0.3) (layer "F.Cu") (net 47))
 (segment (start 76.5 86.6) (end 76.5 83.44) (width 0.3) (layer "F.Cu") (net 47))
 (segment (start 76.5 92) (end 76.5 105.9) (width 0.3) (layer "F.Cu") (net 47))
 (segment (start 76.5 105.9) (end 71.25 111.15) (width 0.3) (layer "F.Cu") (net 47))
 (via (at 76.5 92) (size 0.8) (drill 0.4) (layers "F.Cu" "B.Cu") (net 47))
 (via (at 76.5 86.6) (size 0.8) (drill 0.4) (layers "F.Cu" "B.Cu") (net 47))
 (segment (start 76.5 92) (end 76.5 86.6) (width 0.3) (layer "B.Cu") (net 47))
 (segment (start 80.25 119.5) (end 80.25 92.39) (width 0.3) (layer "F.Cu") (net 15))
 (segment (start 80.25 92.39) (end 80.32 92.32) (width 0.3) (layer "F.Cu") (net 15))
 (segment (start 39.68 74.54) (end 40.5 73.72) (width 0.25) (layer "F.Cu") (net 36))
 (segment (start 40.5 73.72) (end 40.5 73.5) (width 0.25) (layer "F.Cu") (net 36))
 (segment (start 82.86 73.94) (end 82.86 74.54) (width 0.3) (layer "F.Cu") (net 27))
 (segment (start 39.68 84.52) (end 39.68 84.7) (width 0.3) (layer "F.Cu") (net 40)))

